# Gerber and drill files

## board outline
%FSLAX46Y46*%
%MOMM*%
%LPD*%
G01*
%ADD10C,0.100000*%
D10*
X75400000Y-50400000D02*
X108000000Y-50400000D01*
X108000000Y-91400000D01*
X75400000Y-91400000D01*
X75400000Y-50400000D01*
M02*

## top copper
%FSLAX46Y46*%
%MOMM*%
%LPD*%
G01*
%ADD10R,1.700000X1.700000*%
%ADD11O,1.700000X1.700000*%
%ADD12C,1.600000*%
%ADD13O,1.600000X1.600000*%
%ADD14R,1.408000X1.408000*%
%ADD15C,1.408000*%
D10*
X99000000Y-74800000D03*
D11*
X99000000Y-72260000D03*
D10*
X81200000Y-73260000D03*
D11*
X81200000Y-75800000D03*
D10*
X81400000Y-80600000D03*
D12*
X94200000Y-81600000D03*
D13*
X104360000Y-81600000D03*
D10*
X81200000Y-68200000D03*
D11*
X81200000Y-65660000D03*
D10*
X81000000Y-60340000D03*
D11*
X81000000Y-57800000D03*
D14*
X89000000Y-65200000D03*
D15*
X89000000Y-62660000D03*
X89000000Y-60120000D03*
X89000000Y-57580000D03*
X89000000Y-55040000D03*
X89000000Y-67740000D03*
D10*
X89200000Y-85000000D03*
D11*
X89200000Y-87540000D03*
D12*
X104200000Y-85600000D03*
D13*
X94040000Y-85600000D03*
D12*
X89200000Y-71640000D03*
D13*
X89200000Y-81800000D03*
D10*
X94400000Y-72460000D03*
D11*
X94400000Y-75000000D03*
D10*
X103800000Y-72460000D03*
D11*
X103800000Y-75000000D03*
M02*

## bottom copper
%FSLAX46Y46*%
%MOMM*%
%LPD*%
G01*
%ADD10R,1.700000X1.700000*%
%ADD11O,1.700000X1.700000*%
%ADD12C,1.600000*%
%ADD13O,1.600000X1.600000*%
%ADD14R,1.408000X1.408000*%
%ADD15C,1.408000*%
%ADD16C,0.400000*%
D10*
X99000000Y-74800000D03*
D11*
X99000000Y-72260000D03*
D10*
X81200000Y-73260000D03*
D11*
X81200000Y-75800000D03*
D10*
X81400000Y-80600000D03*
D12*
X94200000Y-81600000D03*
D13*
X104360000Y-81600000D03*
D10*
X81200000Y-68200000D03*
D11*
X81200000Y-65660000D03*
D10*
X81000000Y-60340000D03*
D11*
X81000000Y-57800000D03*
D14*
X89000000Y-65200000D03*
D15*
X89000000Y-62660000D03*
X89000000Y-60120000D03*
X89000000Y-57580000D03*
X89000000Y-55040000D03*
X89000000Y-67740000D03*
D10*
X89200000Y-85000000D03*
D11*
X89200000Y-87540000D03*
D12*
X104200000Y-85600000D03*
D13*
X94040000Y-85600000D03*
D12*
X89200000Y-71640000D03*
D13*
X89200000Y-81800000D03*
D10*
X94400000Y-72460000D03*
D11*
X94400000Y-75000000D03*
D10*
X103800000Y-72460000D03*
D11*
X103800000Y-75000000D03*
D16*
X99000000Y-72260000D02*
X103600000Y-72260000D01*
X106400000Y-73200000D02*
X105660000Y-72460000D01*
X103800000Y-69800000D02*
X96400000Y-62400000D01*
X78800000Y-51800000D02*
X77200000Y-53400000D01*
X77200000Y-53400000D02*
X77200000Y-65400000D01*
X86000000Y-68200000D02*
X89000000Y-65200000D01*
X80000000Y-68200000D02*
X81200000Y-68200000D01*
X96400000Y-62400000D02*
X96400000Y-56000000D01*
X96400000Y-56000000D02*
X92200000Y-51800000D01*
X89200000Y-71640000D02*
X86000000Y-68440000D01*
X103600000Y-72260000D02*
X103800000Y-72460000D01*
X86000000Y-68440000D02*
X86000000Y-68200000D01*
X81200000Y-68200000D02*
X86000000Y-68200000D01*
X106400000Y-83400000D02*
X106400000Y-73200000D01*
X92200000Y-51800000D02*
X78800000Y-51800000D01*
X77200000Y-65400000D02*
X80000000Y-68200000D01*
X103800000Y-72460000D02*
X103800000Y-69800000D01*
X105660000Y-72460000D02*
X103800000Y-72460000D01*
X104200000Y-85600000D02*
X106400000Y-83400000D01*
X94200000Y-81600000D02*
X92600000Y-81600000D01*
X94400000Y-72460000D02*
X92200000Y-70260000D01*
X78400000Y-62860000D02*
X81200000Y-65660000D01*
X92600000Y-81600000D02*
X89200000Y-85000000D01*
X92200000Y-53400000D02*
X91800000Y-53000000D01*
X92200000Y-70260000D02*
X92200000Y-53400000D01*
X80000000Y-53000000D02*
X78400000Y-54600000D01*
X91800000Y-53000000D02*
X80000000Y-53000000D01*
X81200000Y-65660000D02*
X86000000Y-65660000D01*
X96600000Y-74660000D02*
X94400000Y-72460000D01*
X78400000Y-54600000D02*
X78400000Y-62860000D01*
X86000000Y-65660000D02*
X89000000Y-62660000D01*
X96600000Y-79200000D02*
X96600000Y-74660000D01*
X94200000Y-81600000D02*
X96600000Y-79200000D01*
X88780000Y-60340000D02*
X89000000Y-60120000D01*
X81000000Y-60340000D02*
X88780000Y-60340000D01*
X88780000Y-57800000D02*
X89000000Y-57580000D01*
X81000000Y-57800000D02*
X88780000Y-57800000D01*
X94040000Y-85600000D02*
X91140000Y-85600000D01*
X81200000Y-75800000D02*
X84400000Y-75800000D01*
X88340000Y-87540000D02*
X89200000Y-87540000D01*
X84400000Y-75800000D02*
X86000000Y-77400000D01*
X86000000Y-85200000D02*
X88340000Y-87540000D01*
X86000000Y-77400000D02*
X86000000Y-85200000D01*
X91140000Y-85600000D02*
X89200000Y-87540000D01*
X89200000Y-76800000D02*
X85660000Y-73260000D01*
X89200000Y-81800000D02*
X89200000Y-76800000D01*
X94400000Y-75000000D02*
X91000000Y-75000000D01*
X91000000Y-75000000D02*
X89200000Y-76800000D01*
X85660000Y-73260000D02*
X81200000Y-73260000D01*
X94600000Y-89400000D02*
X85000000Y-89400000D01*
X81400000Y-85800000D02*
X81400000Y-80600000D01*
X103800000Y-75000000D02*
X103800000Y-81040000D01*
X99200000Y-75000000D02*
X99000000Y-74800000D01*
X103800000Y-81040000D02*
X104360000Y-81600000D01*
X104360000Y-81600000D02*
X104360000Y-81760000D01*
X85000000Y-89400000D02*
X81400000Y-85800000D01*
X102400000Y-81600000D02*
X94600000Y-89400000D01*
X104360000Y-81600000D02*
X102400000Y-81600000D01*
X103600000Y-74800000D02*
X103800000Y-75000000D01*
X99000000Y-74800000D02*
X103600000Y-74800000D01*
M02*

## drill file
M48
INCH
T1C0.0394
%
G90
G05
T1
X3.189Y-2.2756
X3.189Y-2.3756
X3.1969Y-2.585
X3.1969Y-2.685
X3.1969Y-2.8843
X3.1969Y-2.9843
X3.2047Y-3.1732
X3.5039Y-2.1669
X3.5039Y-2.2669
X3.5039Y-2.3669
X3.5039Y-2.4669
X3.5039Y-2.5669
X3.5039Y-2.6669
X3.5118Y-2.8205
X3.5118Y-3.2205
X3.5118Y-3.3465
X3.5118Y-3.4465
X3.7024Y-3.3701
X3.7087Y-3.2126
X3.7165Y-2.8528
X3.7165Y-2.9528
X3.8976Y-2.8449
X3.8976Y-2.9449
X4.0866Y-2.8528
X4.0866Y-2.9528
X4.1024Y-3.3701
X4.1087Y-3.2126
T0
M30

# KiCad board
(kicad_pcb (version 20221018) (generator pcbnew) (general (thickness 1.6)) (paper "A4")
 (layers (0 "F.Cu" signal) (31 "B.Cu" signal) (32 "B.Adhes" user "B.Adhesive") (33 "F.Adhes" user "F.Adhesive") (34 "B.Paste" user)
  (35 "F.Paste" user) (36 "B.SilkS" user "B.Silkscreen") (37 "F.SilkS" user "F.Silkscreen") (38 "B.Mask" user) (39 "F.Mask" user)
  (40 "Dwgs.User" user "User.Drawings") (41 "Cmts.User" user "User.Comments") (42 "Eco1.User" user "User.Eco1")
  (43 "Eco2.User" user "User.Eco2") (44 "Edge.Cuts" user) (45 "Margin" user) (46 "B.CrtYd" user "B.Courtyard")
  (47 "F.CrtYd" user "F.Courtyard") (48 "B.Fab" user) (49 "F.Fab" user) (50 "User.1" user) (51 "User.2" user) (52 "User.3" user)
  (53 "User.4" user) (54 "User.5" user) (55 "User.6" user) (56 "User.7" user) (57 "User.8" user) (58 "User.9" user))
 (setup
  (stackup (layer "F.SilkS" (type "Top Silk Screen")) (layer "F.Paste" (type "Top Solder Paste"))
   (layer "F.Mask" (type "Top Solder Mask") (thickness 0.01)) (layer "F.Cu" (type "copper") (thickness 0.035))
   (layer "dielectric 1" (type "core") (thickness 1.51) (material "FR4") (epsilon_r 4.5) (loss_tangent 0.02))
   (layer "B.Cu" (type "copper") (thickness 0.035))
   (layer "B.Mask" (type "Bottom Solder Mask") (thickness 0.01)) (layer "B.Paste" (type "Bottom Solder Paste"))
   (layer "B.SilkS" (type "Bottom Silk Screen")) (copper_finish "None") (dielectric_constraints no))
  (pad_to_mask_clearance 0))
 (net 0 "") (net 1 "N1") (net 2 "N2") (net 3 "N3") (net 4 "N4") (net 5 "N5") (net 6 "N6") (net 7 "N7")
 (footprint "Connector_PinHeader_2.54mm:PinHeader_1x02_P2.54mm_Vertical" (layer "F.Cu") (at 99 74.8 180)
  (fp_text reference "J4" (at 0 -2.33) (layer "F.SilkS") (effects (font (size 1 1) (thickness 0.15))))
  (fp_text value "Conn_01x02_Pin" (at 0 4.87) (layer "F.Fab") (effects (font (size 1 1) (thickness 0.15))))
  (pad "1" thru_hole rect (at 0 0 180) (size 1.7 1.7) (drill 1) (layers "*.Cu" "*.Mask") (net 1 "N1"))
  (pad "2" thru_hole oval (at 0 2.54 180) (size 1.7 1.7) (drill 1) (layers "*.Cu" "*.Mask") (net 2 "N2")))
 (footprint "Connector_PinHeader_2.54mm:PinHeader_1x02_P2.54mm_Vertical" (layer "F.Cu") (at 81.2 73.26)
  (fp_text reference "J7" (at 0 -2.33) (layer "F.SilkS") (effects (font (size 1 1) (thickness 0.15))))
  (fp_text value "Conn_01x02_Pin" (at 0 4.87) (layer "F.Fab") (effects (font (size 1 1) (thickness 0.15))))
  (pad "1" thru_hole rect (at 0 0) (size 1.7 1.7) (drill 1) (layers "*.Cu" "*.Mask") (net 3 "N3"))
  (pad "2" thru_hole oval (at 0 2.54) (size 1.7 1.7) (drill 1) (layers "*.Cu" "*.Mask") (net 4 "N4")))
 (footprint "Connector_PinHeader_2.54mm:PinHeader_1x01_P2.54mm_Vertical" (layer "F.Cu") (at 81.4 80.6)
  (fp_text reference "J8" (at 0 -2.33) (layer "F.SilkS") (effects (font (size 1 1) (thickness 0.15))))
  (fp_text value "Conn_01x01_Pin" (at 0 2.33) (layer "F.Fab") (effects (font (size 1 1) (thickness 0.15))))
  (pad "1" thru_hole rect (at 0 0) (size 1.7 1.7) (drill 1) (layers "*.Cu" "*.Mask") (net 1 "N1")))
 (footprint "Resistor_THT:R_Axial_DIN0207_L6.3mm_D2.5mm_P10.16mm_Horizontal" (layer "F.Cu") (at 94.2 81.6)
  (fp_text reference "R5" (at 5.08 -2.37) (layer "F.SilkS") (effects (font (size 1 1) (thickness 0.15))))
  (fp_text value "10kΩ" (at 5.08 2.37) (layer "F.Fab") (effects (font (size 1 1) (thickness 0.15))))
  (pad "1" thru_hole circle (at 0 0) (size 1.6 1.6) (drill 1) (layers "*.Cu" "*.Mask") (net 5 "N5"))
  (pad "2" thru_hole oval (at 10.16 0) (size 1.6 1.6) (drill 1) (layers "*.Cu" "*.Mask") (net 1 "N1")))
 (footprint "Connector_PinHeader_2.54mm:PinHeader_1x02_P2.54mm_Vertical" (layer "F.Cu") (at 81.2 68.2 180)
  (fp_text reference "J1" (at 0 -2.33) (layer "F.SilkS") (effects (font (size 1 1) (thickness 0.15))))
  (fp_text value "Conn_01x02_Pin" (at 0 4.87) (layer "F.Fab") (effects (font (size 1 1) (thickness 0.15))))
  (pad "1" thru_hole rect (at 0 0 180) (size 1.7 1.7) (drill 1) (layers "*.Cu" "*.Mask") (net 2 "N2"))
  (pad "2" thru_hole oval (at 0 2.54 180) (size 1.7 1.7) (drill 1) (layers "*.Cu" "*.Mask") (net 5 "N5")))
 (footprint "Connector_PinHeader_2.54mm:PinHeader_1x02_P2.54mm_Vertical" (layer "F.Cu") (at 81 60.34 180)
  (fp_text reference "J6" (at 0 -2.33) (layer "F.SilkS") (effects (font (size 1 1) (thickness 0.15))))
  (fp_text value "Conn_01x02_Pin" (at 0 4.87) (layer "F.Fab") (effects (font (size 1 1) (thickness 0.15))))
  (pad "1" thru_hole rect (at 0 0 180) (size 1.7 1.7) (drill 1) (layers "*.Cu" "*.Mask") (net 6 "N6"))
  (pad "2" thru_hole oval (at 0 2.54 180) (size 1.7 1.7) (drill 1) (layers "*.Cu" "*.Mask") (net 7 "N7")))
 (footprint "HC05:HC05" (layer "F.Cu") (at 89 65.2 180)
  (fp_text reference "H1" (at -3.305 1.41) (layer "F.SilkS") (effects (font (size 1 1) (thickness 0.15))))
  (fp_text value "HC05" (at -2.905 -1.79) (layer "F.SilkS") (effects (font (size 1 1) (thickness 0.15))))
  (pad "1" thru_hole rect (at 0 0 180) (size 1.408 1.408) (drill 1) (layers "*.Cu" "*.Mask") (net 2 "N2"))
  (pad "2" thru_hole circle (at 0 2.54 180) (size 1.408 1.408) (drill 1) (layers "*.Cu" "*.Mask") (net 5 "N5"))
  (pad "3" thru_hole circle (at 0 5.08 180) (size 1.408 1.408) (drill 1) (layers "*.Cu" "*.Mask") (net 6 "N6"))
  (pad "4" thru_hole circle (at 0 7.62 180) (size 1.408 1.408) (drill 1) (layers "*.Cu" "*.Mask") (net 7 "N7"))
  (pad "5" thru_hole circle (at 0 10.16 180) (size 1.408 1.408) (drill 1) (layers "*.Cu" "*.Mask"))
  (pad "6" thru_hole circle (at 0 -2.54 180) (size 1.408 1.408) (drill 1) (layers "*.Cu" "*.Mask")))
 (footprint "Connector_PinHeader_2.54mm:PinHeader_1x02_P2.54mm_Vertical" (layer "F.Cu") (at 89.2 85)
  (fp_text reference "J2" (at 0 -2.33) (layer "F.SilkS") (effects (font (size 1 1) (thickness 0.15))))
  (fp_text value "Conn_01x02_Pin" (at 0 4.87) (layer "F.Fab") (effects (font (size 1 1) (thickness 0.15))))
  (pad "1" thru_hole rect (at 0 0) (size 1.7 1.7) (drill 1) (layers "*.Cu" "*.Mask") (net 5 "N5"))
  (pad "2" thru_hole oval (at 0 2.54) (size 1.7 1.7) (drill 1) (layers "*.Cu" "*.Mask") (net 4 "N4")))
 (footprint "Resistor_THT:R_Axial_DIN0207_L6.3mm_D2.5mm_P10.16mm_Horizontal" (layer "F.Cu") (at 104.2 85.6 180)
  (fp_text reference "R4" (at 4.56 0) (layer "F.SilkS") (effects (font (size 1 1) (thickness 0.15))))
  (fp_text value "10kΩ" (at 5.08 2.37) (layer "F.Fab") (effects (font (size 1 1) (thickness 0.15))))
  (pad "1" thru_hole circle (at 0 0 180) (size 1.6 1.6) (drill 1) (layers "*.Cu" "*.Mask") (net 2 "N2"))
  (pad "2" thru_hole oval (at 10.16 0 180) (size 1.6 1.6) (drill 1) (layers "*.Cu" "*.Mask") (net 4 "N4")))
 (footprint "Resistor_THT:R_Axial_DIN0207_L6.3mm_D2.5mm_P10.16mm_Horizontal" (layer "F.Cu") (at 89.2 71.64 -90)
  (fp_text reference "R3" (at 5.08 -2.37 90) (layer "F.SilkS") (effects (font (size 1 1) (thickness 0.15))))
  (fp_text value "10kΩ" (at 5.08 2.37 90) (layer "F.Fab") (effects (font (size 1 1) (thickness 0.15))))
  (pad "1" thru_hole circle (at 0 0 270) (size 1.6 1.6) (drill 1) (layers "*.Cu" "*.Mask") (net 2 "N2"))
  (pad "2" thru_hole oval (at 10.16 0 270) (size 1.6 1.6) (drill 1) (layers "*.Cu" "*.Mask") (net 3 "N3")))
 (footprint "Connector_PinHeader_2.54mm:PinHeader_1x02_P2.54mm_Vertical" (layer "F.Cu") (at 94.4 72.46)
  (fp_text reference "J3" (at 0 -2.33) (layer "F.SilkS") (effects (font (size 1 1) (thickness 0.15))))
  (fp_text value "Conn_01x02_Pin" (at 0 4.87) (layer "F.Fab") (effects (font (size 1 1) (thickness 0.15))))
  (pad "1" thru_hole rect (at 0 0) (size 1.7 1.7) (drill 1) (layers "*.Cu" "*.Mask") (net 5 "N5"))
  (pad "2" thru_hole oval (at 0 2.54) (size 1.7 1.7) (drill 1) (layers "*.Cu" "*.Mask") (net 3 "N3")))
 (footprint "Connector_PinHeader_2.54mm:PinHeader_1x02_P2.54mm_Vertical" (layer "F.Cu") (at 103.8 72.46)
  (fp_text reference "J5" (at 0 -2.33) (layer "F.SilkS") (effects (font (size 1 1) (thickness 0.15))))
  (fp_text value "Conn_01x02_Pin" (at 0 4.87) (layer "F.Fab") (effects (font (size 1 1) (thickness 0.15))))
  (pad "1" thru_hole rect (at 0 0) (size 1.7 1.7) (drill 1) (layers "*.Cu" "*.Mask") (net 2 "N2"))
  (pad "2" thru_hole oval (at 0 2.54) (size 1.7 1.7) (drill 1) (layers "*.Cu" "*.Mask") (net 1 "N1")))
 (gr_rect (start 75.4 50.4) (end 108 91.4) (stroke (width 0.1) (type default)) (fill none) (layer "Edge.Cuts"))
 (segment (start 99 72.26) (end 103.6 72.26) (width 0.4) (layer "B.Cu") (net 2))
 (segment (start 106.4 73.2) (end 105.66 72.46) (width 0.4) (layer "B.Cu") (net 2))
 (segment (start 103.8 69.8) (end 96.4 62.4) (width 0.4) (layer "B.Cu") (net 2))
 (segment (start 78.8 51.8) (end 77.2 53.4) (width 0.4) (layer "B.Cu") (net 2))
 (segment (start 77.2 53.4) (end 77.2 65.4) (width 0.4) (layer "B.Cu") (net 2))
 (segment (start 86 68.2) (end 89 65.2) (width 0.4) (layer "B.Cu") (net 2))
 (segment (start 80 68.2) (end 81.2 68.2) (width 0.4) (layer "B.Cu") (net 2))
 (segment (start 96.4 62.4) (end 96.4 56) (width 0.4) (layer "B.Cu") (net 2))
 (segment (start 96.4 56) (end 92.2 51.8) (width 0.4) (layer "B.Cu") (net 2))
 (segment (start 89.2 71.64) (end 86 68.44) (width 0.4) (layer "B.Cu") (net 2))
 (segment (start 103.6 72.26) (end 103.8 72.46) (width 0.4) (layer "B.Cu") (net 2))
 (segment (start 86 68.44) (end 86 68.2) (width 0.4) (layer "B.Cu") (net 2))
 (segment (start 81.2 68.2) (end 86 68.2) (width 0.4) (layer "B.Cu") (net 2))
 (segment (start 106.4 83.4) (end 106.4 73.2) (width 0.4) (layer "B.Cu") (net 2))
 (segment (start 92.2 51.8) (end 78.8 51.8) (width 0.4) (layer "B.Cu") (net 2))
 (segment (start 77.2 65.4) (end 80 68.2) (width 0.4) (layer "B.Cu") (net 2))
 (segment (start 103.8 72.46) (end 103.8 69.8) (width 0.4) (layer "B.Cu") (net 2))
 (segment (start 105.66 72.46) (end 103.8 72.46) (width 0.4) (layer "B.Cu") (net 2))
 (segment (start 104.2 85.6) (end 106.4 83.4) (width 0.4) (layer "B.Cu") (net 2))
 (segment (start 94.2 81.6) (end 92.6 81.6) (width 0.4) (layer "B.Cu") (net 5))
 (segment (start 94.4 72.46) (end 92.2 70.26) (width 0.4) (layer "B.Cu") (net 5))
 (segment (start 78.4 62.86) (end 81.2 65.66) (width 0.4) (layer "B.Cu") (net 5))
 (segment (start 92.6 81.6) (end 89.2 85) (width 0.4) (layer "B.Cu") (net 5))
 (segment (start 92.2 53.4) (end 91.8 53) (width 0.4) (layer "B.Cu") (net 5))
 (segment (start 92.2 70.26) (end 92.2 53.4) (width 0.4) (layer "B.Cu") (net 5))
 (segment (start 80 53) (end 78.4 54.6) (width 0.4) (layer "B.Cu") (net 5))
 (segment (start 91.8 53) (end 80 53) (width 0.4) (layer "B.Cu") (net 5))
 (segment (start 81.2 65.66) (end 86 65.66) (width 0.4) (layer "B.Cu") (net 5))
 (segment (start 96.6 74.66) (end 94.4 72.46) (width 0.4) (layer "B.Cu") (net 5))
 (segment (start 78.4 54.6) (end 78.4 62.86) (width 0.4) (layer "B.Cu") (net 5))
 (segment (start 86 65.66) (end 89 62.66) (width 0.4) (layer "B.Cu") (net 5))
 (segment (start 96.6 79.2) (end 96.6 74.66) (width 0.4) (layer "B.Cu") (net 5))
 (segment (start 94.2 81.6) (end 96.6 79.2) (width 0.4) (layer "B.Cu") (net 5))
 (segment (start 88.78 60.34) (end 89 60.12) (width 0.4) (layer "B.Cu") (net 6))
 (segment (start 81 60.34) (end 88.78 60.34) (width 0.4) (layer "B.Cu") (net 6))
 (segment (start 88.78 57.8) (end 89 57.58) (width 0.4) (layer "B.Cu") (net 7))
 (segment (start 81 57.8) (end 88.78 57.8) (width 0.4) (layer "B.Cu") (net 7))
 (segment (start 94.04 85.6) (end 91.14 85.6) (width 0.4) (layer "B.Cu") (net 4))
 (segment (start 81.2 75.8) (end 84.4 75.8) (width 0.4) (layer "B.Cu") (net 4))
 (segment (start 88.34 87.54) (end 89.2 87.54) (width 0.4) (layer "B.Cu") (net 4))
 (segment (start 84.4 75.8) (end 86 77.4) (width 0.4) (layer "B.Cu") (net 4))
 (segment (start 86 85.2) (end 88.34 87.54) (width 0.4) (layer "B.Cu") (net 4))
 (segment (start 86 77.4) (end 86 85.2) (width 0.4) (layer "B.Cu") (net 4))
 (segment (start 91.14 85.6) (end 89.2 87.54) (width 0.4) (layer "B.Cu") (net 4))
 (segment (start 89.2 76.8) (end 85.66 73.26) (width 0.4) (layer "B.Cu") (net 3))
 (segment (start 89.2 81.8) (end 89.2 76.8) (width 0.4) (layer "B.Cu") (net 3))
 (segment (start 94.4 75) (end 91 75) (width 0.4) (layer "B.Cu") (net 3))
 (segment (start 91 75) (end 89.2 76.8) (width 0.4) (layer "B.Cu") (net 3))
 (segment (start 85.66 73.26) (end 81.2 73.26) (width 0.4) (layer "B.Cu") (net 3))
 (segment (start 94.6 89.4) (end 85 89.4) (width 0.4) (layer "B.Cu") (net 1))
 (segment (start 81.4 85.8) (end 81.4 80.6) (width 0.4) (layer "B.Cu") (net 1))
 (segment (start 103.8 75) (end 103.8 81.04) (width 0.4) (layer "B.Cu") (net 1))
 (segment (start 99.2 75) (end 99 74.8) (width 0.4) (layer "B.Cu") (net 1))
 (segment (start 103.8 81.04) (end 104.36 81.6) (width 0.4) (layer "B.Cu") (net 1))
 (segment (start 104.36 81.6) (end 104.36 81.76) (width 0.4) (layer "B.Cu") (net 1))
 (segment (start 85 89.4) (end 81.4 85.8) (width 0.4) (layer "B.Cu") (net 1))
 (segment (start 102.4 81.6) (end 94.6 89.4) (width 0.4) (layer "B.Cu") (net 1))
 (segment (start 104.36 81.6) (end 102.4 81.6) (width 0.4) (layer "B.Cu") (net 1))
 (segment (start 103.6 74.8) (end 103.8 75) (width 0.4) (layer "B.Cu") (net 1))
 (segment (start 99 74.8) (end 103.6 74.8) (width 0.4) (layer "B.Cu") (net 1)))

